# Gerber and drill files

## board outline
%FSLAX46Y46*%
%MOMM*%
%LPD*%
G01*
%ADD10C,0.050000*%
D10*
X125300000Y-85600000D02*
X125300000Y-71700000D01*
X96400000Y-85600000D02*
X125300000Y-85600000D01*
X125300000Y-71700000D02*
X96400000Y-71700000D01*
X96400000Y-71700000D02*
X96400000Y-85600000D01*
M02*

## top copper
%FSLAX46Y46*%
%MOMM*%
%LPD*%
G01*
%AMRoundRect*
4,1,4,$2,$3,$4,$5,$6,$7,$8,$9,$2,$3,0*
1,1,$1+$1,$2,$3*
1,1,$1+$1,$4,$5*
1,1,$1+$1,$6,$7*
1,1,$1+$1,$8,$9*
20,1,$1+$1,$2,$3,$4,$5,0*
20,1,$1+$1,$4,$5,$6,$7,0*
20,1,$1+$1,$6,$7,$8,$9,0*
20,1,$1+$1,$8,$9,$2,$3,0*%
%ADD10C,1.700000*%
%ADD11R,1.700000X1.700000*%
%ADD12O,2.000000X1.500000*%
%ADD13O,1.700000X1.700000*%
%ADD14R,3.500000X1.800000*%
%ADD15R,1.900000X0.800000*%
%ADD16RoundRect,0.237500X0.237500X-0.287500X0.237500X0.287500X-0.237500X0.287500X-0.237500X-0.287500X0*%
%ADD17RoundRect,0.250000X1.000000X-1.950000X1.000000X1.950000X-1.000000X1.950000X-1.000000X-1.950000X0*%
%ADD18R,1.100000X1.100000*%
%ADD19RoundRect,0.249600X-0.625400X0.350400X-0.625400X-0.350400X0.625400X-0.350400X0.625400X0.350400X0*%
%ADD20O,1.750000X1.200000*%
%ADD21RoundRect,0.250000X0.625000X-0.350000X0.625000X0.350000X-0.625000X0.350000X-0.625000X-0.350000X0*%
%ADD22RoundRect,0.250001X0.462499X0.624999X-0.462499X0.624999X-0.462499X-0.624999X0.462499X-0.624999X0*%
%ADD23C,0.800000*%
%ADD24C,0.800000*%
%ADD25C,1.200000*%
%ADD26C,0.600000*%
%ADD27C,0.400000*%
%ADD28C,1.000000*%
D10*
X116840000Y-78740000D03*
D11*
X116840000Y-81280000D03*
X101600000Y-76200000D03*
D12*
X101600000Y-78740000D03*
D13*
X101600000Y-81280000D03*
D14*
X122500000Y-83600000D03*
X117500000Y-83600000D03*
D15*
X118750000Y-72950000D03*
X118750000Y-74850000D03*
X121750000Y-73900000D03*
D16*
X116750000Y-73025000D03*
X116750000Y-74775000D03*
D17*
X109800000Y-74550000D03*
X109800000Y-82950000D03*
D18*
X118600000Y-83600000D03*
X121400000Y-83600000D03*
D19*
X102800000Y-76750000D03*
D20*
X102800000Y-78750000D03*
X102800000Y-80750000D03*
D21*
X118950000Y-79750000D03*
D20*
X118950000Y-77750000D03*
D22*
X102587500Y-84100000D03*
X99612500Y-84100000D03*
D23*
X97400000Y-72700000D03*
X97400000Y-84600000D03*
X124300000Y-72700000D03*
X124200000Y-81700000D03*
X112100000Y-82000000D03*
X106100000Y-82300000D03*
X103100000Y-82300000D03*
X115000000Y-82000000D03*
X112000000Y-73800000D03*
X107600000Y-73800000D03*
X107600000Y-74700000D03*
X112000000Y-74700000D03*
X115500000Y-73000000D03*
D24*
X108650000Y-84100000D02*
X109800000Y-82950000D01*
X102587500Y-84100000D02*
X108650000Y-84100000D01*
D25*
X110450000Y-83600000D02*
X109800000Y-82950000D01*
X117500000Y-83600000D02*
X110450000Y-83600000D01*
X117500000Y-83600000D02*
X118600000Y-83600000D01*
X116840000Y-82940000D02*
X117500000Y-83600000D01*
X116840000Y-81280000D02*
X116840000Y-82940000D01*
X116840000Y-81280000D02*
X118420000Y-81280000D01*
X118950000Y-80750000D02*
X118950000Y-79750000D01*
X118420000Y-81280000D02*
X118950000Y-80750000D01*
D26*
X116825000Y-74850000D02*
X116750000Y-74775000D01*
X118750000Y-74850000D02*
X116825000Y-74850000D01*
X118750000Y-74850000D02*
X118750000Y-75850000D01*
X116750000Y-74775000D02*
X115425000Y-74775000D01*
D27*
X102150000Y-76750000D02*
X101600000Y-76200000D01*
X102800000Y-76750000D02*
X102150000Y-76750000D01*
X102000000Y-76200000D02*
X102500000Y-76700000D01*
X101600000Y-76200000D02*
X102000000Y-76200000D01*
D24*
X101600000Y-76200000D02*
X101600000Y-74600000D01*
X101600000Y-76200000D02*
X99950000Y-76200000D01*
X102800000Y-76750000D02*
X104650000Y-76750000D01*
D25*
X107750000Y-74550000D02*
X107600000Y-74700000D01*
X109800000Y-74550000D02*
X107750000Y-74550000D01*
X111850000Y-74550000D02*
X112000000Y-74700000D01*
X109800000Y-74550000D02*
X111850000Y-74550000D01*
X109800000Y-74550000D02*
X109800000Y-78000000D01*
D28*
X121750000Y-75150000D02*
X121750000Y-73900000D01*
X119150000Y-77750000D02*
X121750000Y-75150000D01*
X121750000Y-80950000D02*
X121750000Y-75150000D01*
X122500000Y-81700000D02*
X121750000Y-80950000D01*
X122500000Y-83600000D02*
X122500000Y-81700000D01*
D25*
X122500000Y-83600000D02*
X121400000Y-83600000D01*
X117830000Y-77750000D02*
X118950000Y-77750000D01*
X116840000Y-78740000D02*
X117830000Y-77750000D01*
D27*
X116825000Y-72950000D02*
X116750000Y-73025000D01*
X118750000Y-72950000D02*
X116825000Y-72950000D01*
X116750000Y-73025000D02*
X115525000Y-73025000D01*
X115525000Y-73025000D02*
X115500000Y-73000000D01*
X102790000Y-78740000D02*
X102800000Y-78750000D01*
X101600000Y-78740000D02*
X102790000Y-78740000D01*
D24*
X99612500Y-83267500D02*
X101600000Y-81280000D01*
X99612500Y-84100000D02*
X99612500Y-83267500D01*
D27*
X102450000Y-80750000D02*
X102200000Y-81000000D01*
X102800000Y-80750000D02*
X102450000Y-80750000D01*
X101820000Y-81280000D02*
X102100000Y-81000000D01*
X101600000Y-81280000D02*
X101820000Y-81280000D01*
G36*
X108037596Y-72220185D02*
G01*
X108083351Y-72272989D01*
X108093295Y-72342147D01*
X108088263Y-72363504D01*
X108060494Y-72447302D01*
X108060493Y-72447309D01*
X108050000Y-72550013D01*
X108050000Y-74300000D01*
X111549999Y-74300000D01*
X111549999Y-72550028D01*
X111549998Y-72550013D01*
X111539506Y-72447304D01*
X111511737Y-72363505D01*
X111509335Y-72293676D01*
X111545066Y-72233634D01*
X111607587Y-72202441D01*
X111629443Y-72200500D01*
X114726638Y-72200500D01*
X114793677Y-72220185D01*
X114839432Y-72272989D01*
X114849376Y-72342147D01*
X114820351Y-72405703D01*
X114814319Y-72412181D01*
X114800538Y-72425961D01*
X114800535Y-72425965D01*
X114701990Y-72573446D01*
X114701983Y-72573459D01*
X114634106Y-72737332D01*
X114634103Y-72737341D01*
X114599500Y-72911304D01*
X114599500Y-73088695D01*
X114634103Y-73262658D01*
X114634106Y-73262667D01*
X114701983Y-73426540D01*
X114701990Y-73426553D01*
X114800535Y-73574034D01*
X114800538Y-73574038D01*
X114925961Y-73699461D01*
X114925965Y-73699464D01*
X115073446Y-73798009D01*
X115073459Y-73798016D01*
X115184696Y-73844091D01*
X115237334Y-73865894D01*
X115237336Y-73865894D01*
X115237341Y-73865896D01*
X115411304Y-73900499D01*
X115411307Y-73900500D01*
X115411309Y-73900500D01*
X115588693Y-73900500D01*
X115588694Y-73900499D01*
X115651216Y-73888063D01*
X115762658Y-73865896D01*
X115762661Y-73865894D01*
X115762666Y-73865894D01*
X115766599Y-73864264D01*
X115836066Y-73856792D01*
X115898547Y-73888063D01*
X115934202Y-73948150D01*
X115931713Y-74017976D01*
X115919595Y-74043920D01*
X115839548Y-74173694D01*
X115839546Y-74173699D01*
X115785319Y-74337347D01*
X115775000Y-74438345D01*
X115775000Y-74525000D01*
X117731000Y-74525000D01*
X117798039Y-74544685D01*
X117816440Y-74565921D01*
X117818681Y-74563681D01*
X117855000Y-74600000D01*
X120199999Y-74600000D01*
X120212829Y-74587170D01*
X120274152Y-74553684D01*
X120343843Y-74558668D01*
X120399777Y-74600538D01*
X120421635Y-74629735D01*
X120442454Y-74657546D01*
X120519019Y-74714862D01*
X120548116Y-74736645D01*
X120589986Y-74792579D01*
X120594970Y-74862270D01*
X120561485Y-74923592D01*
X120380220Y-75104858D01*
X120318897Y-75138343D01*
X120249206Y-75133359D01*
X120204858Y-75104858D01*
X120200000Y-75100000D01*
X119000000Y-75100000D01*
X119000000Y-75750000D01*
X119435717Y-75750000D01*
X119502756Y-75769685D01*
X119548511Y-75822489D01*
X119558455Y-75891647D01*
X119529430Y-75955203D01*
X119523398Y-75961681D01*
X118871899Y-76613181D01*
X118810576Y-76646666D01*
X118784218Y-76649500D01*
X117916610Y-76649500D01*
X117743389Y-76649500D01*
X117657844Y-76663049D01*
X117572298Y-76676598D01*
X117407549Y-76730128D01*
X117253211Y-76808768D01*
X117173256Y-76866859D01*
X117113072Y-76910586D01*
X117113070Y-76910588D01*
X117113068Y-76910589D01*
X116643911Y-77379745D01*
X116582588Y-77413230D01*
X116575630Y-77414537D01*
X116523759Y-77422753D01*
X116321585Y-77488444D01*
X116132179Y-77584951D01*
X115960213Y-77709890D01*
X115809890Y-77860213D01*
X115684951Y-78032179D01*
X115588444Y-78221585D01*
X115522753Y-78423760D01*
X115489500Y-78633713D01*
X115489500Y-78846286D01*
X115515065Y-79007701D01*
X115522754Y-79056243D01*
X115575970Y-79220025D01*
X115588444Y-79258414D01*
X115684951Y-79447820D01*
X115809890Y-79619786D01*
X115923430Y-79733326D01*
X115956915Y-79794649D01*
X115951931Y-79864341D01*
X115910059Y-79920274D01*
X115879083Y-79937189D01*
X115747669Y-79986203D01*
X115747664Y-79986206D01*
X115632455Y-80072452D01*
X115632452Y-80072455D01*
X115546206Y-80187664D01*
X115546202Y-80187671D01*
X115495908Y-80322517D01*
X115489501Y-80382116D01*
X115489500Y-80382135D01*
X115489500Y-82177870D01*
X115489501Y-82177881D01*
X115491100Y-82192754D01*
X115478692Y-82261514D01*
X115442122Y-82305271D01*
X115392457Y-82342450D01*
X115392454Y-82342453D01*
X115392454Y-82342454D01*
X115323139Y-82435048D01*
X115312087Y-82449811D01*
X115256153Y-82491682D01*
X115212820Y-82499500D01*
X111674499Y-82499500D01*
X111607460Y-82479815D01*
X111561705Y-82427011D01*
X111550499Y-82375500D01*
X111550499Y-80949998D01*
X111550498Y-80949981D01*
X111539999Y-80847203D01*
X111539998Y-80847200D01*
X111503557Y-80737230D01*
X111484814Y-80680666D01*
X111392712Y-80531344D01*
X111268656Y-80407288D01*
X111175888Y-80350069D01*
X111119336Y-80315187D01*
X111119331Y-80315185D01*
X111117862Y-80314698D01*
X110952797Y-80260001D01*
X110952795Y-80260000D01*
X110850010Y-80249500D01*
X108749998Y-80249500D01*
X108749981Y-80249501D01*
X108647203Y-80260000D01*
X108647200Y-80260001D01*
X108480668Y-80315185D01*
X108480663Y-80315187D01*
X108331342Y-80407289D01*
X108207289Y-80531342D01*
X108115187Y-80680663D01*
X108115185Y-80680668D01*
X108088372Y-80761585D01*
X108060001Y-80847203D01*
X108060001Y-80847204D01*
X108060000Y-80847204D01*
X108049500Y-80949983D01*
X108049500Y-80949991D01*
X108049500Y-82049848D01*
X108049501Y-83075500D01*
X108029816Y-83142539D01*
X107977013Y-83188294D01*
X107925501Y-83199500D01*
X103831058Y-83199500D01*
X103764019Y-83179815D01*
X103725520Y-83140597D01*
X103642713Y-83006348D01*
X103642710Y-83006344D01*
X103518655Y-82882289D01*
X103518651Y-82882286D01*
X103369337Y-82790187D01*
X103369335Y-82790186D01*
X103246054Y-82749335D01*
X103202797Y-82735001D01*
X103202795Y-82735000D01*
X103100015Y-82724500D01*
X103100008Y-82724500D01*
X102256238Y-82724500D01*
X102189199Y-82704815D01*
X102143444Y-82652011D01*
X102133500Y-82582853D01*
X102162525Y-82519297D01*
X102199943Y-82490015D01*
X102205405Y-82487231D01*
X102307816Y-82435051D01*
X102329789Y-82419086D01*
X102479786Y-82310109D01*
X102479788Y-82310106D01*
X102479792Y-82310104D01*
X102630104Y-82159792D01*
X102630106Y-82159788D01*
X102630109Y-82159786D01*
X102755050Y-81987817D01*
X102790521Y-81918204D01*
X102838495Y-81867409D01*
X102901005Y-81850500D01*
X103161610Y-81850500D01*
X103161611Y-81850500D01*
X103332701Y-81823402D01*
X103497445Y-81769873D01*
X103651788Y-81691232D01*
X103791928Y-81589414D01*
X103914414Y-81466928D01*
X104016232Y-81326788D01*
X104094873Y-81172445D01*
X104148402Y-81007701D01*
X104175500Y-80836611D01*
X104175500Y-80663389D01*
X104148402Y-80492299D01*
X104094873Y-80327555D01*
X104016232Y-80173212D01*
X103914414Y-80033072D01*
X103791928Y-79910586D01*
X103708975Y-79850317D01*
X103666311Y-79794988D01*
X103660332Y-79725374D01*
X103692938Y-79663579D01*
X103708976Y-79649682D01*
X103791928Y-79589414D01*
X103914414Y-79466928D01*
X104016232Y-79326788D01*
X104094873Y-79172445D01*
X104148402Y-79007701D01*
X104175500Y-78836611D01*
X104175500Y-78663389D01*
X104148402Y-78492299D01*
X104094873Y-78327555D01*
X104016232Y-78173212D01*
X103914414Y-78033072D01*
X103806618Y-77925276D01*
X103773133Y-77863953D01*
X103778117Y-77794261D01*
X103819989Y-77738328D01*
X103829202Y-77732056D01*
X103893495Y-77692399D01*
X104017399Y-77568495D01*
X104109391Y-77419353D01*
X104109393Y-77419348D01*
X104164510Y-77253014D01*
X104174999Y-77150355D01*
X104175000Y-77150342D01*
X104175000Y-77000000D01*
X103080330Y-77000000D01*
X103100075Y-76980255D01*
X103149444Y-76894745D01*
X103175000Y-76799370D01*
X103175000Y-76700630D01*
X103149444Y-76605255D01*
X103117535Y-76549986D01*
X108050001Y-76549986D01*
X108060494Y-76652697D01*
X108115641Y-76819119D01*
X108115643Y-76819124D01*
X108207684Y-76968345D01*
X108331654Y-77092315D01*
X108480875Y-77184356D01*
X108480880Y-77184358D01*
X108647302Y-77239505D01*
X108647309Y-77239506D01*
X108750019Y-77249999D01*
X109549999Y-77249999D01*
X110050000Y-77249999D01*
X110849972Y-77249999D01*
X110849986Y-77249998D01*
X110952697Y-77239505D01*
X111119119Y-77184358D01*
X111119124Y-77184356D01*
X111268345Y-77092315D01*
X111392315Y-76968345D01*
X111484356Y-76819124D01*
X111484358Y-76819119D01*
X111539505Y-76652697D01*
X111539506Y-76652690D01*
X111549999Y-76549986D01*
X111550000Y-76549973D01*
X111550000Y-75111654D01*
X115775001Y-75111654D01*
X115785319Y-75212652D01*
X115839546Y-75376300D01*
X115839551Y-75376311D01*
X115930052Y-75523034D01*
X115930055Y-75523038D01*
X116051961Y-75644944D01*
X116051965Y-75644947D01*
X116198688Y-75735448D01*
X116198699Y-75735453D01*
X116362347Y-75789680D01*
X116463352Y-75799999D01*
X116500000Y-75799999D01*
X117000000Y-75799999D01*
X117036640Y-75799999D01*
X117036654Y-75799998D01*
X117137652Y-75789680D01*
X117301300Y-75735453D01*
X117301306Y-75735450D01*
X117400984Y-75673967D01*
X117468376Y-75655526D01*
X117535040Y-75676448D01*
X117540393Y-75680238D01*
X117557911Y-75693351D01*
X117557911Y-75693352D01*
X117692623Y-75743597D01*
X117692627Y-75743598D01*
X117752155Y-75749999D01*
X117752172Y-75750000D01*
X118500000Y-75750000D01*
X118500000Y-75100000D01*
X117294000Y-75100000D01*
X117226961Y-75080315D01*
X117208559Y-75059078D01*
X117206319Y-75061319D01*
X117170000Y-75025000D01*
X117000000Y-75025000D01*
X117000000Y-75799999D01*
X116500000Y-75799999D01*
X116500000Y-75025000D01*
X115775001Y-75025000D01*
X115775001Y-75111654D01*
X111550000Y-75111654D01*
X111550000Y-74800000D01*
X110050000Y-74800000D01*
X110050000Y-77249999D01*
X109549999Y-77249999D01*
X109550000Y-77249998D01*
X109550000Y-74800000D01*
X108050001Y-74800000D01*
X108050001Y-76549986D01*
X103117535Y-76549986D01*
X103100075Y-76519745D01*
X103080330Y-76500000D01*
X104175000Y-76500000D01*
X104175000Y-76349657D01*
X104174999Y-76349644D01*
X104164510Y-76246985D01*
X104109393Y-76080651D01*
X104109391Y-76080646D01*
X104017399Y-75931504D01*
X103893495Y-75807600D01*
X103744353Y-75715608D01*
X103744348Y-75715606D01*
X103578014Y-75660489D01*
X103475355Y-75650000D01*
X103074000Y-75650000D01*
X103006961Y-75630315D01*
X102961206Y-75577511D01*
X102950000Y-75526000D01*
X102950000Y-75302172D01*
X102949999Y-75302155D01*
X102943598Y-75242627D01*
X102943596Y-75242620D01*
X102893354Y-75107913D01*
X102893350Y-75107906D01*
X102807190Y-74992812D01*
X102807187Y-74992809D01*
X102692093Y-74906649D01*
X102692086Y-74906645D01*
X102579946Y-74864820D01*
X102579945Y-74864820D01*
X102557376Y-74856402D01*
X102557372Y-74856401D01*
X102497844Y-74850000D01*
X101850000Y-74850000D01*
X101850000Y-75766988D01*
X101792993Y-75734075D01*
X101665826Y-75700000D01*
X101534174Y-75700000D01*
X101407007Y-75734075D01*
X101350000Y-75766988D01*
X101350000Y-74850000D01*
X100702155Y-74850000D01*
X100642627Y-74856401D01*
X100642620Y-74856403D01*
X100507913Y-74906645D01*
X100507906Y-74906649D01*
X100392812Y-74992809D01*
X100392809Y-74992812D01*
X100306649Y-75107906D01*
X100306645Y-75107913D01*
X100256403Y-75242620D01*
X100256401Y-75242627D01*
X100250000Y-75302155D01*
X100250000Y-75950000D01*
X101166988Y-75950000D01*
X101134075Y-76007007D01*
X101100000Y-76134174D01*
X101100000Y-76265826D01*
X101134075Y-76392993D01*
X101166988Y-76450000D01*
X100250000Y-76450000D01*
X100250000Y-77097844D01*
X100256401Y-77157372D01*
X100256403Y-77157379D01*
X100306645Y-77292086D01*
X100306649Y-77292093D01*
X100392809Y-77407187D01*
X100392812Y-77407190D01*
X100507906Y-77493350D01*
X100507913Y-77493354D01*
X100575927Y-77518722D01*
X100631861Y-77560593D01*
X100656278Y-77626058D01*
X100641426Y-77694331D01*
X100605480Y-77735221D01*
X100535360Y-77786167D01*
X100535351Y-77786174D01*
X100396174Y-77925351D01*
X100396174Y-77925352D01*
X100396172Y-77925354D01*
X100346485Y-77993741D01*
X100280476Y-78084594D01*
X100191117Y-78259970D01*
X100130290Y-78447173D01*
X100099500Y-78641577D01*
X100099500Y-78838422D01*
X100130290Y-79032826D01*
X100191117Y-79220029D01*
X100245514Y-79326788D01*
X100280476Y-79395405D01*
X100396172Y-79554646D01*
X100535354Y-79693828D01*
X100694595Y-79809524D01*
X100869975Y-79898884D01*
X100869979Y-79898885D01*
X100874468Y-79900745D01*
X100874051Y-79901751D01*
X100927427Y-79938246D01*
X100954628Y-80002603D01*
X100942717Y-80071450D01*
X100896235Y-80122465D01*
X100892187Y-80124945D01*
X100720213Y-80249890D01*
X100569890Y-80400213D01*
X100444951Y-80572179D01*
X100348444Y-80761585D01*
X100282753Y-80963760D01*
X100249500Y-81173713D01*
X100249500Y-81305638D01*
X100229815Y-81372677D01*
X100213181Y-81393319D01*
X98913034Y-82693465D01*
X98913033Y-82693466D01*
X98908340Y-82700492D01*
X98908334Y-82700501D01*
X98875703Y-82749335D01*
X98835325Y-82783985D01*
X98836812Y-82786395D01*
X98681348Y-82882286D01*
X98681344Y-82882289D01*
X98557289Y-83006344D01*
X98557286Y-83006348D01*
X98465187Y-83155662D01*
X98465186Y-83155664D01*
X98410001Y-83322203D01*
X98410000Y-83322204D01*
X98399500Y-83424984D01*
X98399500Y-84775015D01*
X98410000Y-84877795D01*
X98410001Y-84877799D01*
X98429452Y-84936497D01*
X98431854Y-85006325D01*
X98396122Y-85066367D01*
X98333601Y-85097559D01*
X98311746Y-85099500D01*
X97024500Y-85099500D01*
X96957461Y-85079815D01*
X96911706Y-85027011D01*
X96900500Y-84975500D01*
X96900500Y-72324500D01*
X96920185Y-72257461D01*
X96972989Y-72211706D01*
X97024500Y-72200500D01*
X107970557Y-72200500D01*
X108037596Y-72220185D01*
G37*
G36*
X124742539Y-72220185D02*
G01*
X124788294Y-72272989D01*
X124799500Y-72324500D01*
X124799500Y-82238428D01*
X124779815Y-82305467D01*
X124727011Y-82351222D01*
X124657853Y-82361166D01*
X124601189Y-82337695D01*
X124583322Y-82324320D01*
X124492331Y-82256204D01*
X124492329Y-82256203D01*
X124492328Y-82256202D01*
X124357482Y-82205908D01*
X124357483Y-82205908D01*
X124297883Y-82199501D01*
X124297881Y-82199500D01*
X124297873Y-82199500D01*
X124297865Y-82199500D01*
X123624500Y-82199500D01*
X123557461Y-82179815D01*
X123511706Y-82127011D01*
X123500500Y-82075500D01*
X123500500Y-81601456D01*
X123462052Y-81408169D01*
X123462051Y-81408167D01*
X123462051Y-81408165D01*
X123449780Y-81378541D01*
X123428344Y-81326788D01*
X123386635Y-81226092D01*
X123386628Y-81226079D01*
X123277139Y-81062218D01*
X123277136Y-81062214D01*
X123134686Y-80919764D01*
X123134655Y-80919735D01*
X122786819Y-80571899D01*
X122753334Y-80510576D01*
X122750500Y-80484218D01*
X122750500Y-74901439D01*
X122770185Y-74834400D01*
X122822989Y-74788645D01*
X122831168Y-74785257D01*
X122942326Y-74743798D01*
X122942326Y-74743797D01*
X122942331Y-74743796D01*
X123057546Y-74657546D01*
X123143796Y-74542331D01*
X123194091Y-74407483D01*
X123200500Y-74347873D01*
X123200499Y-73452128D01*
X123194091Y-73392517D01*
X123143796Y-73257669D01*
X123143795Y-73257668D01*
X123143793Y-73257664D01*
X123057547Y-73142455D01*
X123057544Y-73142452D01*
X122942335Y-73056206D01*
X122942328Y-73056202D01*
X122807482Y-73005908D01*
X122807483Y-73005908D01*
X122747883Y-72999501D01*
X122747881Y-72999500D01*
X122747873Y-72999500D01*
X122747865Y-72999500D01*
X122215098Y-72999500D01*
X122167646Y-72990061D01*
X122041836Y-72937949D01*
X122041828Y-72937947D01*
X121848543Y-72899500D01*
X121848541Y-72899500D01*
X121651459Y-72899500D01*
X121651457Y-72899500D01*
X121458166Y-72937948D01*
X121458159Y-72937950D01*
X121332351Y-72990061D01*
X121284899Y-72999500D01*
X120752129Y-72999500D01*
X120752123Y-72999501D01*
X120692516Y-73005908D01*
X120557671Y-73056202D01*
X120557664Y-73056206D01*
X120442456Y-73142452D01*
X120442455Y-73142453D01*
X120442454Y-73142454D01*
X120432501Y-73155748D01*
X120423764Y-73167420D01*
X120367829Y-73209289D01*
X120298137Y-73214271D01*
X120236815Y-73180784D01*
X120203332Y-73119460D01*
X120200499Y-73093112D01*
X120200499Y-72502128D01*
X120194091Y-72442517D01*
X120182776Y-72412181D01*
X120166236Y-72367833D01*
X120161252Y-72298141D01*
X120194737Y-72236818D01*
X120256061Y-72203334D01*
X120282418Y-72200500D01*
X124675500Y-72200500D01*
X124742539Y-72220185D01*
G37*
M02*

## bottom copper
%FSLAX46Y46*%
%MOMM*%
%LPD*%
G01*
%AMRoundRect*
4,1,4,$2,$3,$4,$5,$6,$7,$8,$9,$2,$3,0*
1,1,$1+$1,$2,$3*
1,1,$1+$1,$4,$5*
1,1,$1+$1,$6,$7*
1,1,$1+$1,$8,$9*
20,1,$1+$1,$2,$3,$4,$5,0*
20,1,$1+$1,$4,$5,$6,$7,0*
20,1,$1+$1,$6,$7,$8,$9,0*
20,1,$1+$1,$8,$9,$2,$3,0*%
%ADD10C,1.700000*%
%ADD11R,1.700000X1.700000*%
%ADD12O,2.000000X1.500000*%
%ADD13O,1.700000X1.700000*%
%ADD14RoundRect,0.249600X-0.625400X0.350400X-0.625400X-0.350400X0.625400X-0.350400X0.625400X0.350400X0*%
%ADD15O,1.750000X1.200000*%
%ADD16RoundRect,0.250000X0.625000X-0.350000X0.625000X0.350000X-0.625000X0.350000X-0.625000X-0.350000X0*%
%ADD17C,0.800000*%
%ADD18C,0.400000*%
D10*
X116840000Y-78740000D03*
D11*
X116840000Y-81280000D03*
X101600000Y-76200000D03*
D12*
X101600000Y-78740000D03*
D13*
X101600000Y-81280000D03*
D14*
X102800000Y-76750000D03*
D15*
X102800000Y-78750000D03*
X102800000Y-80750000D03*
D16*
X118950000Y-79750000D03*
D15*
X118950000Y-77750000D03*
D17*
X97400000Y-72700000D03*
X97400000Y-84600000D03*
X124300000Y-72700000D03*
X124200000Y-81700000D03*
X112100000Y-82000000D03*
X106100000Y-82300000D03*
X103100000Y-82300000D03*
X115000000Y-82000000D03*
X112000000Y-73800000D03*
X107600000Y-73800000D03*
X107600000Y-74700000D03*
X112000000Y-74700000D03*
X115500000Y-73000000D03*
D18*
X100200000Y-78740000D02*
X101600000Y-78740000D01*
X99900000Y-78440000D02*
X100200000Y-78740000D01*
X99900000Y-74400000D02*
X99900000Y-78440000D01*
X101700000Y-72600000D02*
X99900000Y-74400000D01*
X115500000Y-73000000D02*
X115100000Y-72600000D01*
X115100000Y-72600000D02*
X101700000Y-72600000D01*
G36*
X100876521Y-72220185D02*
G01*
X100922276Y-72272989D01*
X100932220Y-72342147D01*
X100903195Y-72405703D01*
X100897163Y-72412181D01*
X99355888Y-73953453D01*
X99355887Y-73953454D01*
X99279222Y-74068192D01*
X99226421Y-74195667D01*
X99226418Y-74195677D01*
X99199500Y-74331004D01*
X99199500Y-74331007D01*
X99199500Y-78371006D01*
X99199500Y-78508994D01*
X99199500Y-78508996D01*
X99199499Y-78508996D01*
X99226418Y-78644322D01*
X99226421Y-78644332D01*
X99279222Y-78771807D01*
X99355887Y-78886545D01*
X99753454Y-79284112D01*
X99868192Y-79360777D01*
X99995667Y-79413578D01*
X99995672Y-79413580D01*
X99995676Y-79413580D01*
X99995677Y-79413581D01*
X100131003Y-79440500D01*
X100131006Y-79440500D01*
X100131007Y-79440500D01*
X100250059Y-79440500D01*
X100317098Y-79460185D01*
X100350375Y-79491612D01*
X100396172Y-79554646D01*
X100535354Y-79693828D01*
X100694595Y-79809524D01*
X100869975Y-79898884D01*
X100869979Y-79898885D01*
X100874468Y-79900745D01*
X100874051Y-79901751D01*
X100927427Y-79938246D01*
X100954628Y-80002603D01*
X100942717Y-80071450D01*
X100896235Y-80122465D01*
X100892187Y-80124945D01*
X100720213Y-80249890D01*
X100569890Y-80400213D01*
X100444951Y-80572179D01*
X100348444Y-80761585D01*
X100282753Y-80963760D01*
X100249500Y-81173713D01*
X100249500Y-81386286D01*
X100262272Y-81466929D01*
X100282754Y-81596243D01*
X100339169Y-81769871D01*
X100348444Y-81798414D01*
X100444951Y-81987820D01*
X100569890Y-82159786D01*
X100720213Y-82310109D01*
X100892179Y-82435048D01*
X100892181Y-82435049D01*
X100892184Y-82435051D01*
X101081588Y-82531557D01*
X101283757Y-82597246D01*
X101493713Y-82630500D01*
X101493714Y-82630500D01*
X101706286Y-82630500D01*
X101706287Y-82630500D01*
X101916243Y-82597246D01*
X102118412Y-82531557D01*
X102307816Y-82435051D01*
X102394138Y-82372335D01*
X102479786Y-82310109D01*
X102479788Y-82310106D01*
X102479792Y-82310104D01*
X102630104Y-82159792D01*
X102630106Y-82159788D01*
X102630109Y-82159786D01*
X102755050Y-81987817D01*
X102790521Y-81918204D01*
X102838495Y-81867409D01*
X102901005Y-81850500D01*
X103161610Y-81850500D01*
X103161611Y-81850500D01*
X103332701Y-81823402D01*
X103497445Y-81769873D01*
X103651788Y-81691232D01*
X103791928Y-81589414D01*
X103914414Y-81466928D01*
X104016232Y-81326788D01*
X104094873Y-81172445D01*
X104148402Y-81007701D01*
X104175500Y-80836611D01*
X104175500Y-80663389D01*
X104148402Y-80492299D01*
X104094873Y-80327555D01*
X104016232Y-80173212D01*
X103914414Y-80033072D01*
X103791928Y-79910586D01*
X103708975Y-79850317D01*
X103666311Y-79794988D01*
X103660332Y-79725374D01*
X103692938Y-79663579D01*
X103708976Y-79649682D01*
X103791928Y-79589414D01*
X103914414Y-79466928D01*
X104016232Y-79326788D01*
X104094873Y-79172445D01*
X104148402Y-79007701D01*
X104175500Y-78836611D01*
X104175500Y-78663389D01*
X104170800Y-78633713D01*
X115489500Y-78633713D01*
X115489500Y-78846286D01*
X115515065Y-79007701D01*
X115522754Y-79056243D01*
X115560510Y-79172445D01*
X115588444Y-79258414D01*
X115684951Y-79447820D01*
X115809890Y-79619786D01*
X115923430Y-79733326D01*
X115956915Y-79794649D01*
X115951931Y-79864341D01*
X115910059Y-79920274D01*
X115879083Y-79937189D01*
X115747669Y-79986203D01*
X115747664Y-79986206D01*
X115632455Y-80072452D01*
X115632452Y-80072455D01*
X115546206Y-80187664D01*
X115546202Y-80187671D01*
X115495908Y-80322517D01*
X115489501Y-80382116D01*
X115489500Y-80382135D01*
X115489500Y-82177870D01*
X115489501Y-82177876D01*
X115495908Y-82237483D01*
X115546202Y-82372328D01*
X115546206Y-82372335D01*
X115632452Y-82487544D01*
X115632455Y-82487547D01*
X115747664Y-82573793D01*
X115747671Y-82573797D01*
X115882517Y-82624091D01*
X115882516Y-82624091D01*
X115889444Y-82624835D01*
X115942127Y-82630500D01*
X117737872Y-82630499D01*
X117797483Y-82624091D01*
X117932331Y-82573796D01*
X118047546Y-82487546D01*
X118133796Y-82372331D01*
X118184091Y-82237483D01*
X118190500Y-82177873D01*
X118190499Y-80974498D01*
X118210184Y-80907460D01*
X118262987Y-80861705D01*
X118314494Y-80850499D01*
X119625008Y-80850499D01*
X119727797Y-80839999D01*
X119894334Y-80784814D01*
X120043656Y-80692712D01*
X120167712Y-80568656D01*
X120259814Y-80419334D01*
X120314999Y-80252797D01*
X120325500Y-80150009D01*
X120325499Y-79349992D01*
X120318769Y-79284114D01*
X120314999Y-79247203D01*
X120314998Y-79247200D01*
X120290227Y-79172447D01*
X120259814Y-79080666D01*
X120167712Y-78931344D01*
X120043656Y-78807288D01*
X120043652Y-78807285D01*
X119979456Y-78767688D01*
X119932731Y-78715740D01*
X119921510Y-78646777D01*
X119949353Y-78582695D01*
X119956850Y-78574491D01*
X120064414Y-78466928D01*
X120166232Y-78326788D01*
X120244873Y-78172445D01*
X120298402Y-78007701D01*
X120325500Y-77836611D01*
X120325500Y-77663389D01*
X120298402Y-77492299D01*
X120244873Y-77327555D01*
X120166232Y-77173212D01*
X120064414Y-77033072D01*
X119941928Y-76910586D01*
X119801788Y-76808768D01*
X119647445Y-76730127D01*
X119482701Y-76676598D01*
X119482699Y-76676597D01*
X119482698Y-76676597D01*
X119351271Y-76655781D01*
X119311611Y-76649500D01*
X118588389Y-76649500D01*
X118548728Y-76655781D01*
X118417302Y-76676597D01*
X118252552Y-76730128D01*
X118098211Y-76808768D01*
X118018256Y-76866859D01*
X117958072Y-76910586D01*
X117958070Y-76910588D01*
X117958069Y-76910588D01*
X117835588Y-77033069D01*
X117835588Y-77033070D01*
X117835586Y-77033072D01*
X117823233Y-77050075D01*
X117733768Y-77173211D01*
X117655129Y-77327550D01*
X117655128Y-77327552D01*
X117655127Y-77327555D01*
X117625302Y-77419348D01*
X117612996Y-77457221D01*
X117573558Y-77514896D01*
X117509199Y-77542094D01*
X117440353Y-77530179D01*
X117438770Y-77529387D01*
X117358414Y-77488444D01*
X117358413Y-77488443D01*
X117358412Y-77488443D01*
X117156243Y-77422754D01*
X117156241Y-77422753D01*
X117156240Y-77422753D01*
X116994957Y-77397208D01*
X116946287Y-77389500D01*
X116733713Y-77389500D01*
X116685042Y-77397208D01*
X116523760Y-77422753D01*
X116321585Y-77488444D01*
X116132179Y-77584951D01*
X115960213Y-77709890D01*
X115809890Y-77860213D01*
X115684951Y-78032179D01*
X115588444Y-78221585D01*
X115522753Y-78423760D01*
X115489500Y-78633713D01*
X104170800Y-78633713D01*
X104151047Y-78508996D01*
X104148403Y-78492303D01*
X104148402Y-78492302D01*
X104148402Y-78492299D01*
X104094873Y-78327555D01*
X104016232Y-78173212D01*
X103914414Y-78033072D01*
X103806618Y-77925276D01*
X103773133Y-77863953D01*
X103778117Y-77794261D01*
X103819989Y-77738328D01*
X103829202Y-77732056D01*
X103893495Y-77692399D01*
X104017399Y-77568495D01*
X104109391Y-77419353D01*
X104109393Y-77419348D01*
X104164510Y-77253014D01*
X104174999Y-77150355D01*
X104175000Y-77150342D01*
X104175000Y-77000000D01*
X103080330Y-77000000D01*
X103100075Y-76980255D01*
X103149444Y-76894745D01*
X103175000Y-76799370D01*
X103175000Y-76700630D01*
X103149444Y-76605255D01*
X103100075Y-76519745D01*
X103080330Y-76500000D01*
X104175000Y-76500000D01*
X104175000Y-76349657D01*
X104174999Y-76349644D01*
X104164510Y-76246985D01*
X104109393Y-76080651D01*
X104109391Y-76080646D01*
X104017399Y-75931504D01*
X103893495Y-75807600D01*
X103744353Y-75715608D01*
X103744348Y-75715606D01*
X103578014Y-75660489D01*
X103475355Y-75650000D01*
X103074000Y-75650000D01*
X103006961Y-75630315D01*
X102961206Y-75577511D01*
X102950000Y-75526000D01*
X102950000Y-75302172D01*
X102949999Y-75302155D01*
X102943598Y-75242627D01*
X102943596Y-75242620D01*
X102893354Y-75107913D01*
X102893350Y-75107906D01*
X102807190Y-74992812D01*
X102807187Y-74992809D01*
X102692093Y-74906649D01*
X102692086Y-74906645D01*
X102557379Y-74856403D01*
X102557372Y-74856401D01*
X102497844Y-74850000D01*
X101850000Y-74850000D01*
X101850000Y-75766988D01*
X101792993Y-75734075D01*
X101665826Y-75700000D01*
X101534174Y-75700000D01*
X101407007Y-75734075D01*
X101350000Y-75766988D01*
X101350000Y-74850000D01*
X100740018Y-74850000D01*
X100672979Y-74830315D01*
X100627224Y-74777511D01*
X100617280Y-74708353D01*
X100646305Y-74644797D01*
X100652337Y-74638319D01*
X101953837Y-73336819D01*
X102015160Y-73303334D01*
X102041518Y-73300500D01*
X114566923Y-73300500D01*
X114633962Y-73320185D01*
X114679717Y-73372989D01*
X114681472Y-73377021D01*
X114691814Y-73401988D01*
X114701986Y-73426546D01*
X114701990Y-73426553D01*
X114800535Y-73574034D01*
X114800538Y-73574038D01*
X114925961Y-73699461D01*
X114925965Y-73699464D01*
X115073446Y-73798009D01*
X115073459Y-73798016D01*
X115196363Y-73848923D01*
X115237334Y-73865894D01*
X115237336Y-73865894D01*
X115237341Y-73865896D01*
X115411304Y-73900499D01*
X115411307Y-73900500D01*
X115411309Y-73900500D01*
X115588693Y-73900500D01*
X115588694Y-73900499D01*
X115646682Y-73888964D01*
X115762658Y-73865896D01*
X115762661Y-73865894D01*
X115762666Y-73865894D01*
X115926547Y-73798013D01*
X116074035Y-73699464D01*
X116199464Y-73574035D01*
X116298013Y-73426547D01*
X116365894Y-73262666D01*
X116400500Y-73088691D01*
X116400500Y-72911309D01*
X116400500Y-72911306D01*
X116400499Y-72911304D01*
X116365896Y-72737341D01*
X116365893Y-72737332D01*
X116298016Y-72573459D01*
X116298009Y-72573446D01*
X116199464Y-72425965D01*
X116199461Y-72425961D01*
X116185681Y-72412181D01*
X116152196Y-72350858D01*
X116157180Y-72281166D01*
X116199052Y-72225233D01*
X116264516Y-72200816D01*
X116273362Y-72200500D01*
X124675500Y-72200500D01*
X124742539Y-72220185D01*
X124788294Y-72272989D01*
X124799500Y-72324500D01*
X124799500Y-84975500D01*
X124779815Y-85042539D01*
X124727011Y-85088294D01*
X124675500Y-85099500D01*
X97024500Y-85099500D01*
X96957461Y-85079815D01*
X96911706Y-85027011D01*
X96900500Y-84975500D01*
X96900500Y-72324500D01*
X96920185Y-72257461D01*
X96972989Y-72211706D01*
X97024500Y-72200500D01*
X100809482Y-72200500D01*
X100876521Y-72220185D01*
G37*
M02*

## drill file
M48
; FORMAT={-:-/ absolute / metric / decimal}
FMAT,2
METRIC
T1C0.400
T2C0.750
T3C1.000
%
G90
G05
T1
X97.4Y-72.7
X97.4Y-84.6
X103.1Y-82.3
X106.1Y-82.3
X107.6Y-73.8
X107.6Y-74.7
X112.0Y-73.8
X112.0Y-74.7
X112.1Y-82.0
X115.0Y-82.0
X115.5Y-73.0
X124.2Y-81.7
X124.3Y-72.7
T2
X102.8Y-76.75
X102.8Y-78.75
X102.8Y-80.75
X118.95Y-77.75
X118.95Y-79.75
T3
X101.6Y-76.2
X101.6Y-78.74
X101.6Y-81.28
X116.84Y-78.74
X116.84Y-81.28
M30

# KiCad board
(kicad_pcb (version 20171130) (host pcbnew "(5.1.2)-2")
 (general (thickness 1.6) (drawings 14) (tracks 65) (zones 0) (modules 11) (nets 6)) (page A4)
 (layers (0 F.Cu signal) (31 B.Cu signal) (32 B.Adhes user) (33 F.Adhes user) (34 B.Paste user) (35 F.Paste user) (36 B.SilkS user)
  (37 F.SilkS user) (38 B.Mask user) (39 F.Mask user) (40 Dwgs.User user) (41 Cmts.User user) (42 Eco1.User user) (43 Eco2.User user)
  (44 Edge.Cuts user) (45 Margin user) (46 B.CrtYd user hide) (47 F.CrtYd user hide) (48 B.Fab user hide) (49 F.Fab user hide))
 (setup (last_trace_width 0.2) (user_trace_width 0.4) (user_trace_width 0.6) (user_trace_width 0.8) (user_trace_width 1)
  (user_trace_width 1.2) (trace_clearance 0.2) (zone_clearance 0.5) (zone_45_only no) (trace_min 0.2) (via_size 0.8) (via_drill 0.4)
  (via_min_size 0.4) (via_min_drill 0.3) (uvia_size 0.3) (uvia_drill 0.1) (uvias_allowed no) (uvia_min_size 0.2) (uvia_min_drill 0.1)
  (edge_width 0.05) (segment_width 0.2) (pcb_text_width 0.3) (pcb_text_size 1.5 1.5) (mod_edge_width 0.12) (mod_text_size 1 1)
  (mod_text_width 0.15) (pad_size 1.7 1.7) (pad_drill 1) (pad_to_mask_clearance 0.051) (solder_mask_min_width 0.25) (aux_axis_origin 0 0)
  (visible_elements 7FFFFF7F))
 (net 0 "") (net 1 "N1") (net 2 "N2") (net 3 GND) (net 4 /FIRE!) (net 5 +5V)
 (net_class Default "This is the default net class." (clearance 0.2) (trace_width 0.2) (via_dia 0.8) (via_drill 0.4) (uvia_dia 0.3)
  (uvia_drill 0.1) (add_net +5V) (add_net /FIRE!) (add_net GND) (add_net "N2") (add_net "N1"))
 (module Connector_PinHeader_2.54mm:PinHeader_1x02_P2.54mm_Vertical (layer F.Cu) (at 116.84 81.28 180)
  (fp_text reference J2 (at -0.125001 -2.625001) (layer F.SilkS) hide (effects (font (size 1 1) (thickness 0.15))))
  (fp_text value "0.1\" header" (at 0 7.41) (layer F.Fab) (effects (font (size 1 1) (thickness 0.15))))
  (pad 2 thru_hole circle (at 0 2.54 180) (size 1.7 1.7) (drill 1) (layers *.Cu *.Mask) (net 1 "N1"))
  (pad 1 thru_hole rect (at 0 0 180) (size 1.7 1.7) (drill 1) (layers *.Cu *.Mask) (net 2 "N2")))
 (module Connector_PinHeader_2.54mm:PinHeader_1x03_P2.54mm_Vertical (layer F.Cu) (at 101.6 76.2)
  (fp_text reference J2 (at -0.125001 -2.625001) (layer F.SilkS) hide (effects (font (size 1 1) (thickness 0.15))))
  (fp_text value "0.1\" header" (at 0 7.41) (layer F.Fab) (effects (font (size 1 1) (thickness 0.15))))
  (pad 1 thru_hole rect (at 0 0 90) (size 1.7 1.7) (drill 1) (layers *.Cu *.Mask) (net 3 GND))
  (pad 2 thru_hole oval (at 0 2.54) (size 2 1.5) (drill 1) (layers *.Cu *.Mask) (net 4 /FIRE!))
  (pad 3 thru_hole oval (at 0 5.08) (size 1.7 1.7) (drill 1) (layers *.Cu *.Mask) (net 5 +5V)))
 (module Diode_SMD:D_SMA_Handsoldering (layer F.Cu) (at 120 83.6)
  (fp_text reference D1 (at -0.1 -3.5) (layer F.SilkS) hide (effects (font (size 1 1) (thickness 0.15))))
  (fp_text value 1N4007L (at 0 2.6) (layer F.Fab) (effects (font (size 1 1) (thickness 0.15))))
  (pad 2 smd rect (at 2.5 0) (size 3.5 1.8) (layers F.Cu F.Paste F.Mask) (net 1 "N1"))
  (pad 1 smd rect (at -2.5 0) (size 3.5 1.8) (layers F.Cu F.Paste F.Mask) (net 2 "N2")))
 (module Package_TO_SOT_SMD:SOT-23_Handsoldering (layer F.Cu) (at 120.25 73.9)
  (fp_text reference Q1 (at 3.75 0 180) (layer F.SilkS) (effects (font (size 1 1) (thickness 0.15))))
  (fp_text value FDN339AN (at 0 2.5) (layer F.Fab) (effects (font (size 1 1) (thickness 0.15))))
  (pad 1 smd rect (at -1.5 -0.95) (size 1.9 0.8) (layers F.Cu F.Paste F.Mask) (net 4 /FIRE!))
  (pad 2 smd rect (at -1.5 0.95) (size 1.9 0.8) (layers F.Cu F.Paste F.Mask) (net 3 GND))
  (pad 3 smd rect (at 1.5 0) (size 1.9 0.8) (layers F.Cu F.Paste F.Mask) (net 1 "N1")))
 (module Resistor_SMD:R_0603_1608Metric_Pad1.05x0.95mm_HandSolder (layer F.Cu) (at 116.75 73.9 90)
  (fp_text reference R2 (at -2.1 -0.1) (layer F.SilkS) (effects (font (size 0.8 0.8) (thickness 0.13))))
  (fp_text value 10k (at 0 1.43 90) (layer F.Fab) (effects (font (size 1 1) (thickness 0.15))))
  (pad 2 smd roundrect (at 0.875 0 90) (size 1.05 0.95) (layers F.Cu F.Paste F.Mask) (roundrect_rratio 0.25) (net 4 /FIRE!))
  (pad 1 smd roundrect (at -0.875 0 90) (size 1.05 0.95) (layers F.Cu F.Paste F.Mask) (roundrect_rratio 0.25) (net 3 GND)))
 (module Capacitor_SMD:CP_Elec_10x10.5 (layer F.Cu) (at 109.8 78.75 90)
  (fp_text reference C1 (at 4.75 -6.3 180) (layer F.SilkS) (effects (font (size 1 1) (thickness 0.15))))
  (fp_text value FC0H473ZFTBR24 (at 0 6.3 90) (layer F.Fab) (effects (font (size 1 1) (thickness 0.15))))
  (pad 2 smd roundrect (at 4.2 0 90) (size 4.4 2.5) (layers F.Cu F.Paste F.Mask) (roundrect_rratio 0.1) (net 3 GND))
  (pad 1 smd roundrect (at -4.2 0 90) (size 4.4 2.5) (layers F.Cu F.Paste F.Mask) (roundrect_rratio 0.1) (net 2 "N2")))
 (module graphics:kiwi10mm (layer B.Cu) (at 109.6 79.1 180)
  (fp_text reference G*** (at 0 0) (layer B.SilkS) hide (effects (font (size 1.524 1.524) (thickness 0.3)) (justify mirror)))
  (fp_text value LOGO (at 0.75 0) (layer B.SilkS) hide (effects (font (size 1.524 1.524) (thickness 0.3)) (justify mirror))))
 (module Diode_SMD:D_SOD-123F (layer F.Cu) (at 120 83.6)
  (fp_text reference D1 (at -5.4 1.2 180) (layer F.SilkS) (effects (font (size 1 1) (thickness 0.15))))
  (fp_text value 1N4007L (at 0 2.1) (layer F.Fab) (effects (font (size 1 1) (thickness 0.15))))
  (pad 1 smd rect (at -1.4 0) (size 1.1 1.1) (layers F.Cu F.Paste F.Mask) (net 2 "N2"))
  (pad 2 smd rect (at 1.4 0) (size 1.1 1.1) (layers F.Cu F.Paste F.Mask) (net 1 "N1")))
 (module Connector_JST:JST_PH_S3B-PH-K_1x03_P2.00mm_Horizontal (layer F.Cu) (at 102.8 76.75 270)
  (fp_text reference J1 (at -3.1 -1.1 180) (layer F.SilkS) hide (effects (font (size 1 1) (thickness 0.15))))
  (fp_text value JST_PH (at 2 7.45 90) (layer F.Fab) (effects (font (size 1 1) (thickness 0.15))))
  (pad 1 thru_hole roundrect (at 0 0 270) (size 1.2 1.75) (drill 0.75) (layers *.Cu *.Mask) (roundrect_rratio 0.208) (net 3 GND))
  (pad 2 thru_hole oval (at 2 0 270) (size 1.2 1.75) (drill 0.75) (layers *.Cu *.Mask) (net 4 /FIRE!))
  (pad 3 thru_hole oval (at 4 0 270) (size 1.2 1.75) (drill 0.75) (layers *.Cu *.Mask) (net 5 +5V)))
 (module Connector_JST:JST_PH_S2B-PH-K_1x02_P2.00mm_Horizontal (layer F.Cu) (at 118.95 79.75 90)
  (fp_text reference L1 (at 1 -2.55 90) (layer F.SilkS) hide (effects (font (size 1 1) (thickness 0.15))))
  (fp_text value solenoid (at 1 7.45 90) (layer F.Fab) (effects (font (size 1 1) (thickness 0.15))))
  (pad 1 thru_hole roundrect (at 0 0 90) (size 1.2 1.75) (drill 0.75) (layers *.Cu *.Mask) (roundrect_rratio 0.208333) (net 2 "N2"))
  (pad 2 thru_hole oval (at 2 0 90) (size 1.2 1.75) (drill 0.75) (layers *.Cu *.Mask) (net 1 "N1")))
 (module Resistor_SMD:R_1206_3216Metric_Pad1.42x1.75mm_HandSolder (layer F.Cu) (at 101.1 84.1 180)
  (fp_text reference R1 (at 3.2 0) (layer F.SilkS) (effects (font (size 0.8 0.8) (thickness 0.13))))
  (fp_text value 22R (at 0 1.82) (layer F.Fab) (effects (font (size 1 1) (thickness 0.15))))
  (pad 1 smd roundrect (at -1.4875 0 180) (size 1.425 1.75) (layers F.Cu F.Paste F.Mask) (roundrect_rratio 0.175439) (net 2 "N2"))
  (pad 2 smd roundrect (at 1.4875 0 180) (size 1.425 1.75) (layers F.Cu F.Paste F.Mask) (roundrect_rratio 0.175439) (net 5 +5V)))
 (gr_line (start 125.3 85.6) (end 125.3 71.7) (layer Edge.Cuts) (width 0.05))
 (gr_line (start 96.4 85.6) (end 125.3 85.6) (layer Edge.Cuts) (width 0.05))
 (gr_line (start 125.3 71.7) (end 96.4 71.7) (layer Edge.Cuts) (width 0.05))
 (gr_line (start 96.4 71.7) (end 96.4 85.6) (layer Edge.Cuts) (width 0.05))
 (segment (start 108.65 84.1) (end 109.8 82.95) (width 0.8) (layer F.Cu) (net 2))
 (segment (start 102.5875 84.1) (end 108.65 84.1) (width 0.8) (layer F.Cu) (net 2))
 (segment (start 110.45 83.6) (end 109.8 82.95) (width 1.2) (layer F.Cu) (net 2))
 (segment (start 117.5 83.6) (end 110.45 83.6) (width 1.2) (layer F.Cu) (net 2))
 (segment (start 117.5 83.6) (end 118.6 83.6) (width 1.2) (layer F.Cu) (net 2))
 (segment (start 116.84 82.94) (end 117.5 83.6) (width 1.2) (layer F.Cu) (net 2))
 (segment (start 116.84 81.28) (end 116.84 82.94) (width 1.2) (layer F.Cu) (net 2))
 (segment (start 116.84 81.28) (end 118.42 81.28) (width 1.2) (layer F.Cu) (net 2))
 (segment (start 118.95 80.75) (end 118.95 79.75) (width 1.2) (layer F.Cu) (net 2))
 (segment (start 118.42 81.28) (end 118.95 80.75) (width 1.2) (layer F.Cu) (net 2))
 (segment (start 116.825 74.85) (end 116.75 74.775) (width 0.6) (layer F.Cu) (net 3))
 (segment (start 118.75 74.85) (end 116.825 74.85) (width 0.6) (layer F.Cu) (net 3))
 (segment (start 118.75 74.85) (end 118.75 75.85) (width 0.6) (layer F.Cu) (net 3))
 (segment (start 116.75 74.775) (end 115.425 74.775) (width 0.6) (layer F.Cu) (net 3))
 (segment (start 102.15 76.75) (end 101.6 76.2) (width 0.4) (layer F.Cu) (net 3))
 (segment (start 102.8 76.75) (end 102.15 76.75) (width 0.4) (layer F.Cu) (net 3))
 (via (at 97.4 72.7) (size 0.8) (drill 0.4) (layers F.Cu B.Cu) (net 3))
 (via (at 97.4 84.6) (size 0.8) (drill 0.4) (layers F.Cu B.Cu) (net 3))
 (via (at 124.3 72.7) (size 0.8) (drill 0.4) (layers F.Cu B.Cu) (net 3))
 (via (at 124.2 81.7) (size 0.8) (drill 0.4) (layers F.Cu B.Cu) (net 3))
 (via (at 112.1 82) (size 0.8) (drill 0.4) (layers F.Cu B.Cu) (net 3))
 (via (at 106.1 82.3) (size 0.8) (drill 0.4) (layers F.Cu B.Cu) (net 3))
 (via (at 103.1 82.3) (size 0.8) (drill 0.4) (layers F.Cu B.Cu) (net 3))
 (segment (start 102 76.2) (end 102.5 76.7) (width 0.4) (layer F.Cu) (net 3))
 (segment (start 101.6 76.2) (end 102 76.2) (width 0.4) (layer F.Cu) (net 3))
 (segment (start 101.6 76.2) (end 101.6 74.6) (width 0.8) (layer F.Cu) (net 3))
 (segment (start 101.6 76.2) (end 99.95 76.2) (width 0.8) (layer F.Cu) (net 3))
 (segment (start 102.8 76.75) (end 104.65 76.75) (width 0.8) (layer F.Cu) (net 3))
 (via (at 115 82) (size 0.8) (drill 0.4) (layers F.Cu B.Cu) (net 3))
 (via (at 112 73.8) (size 0.8) (drill 0.4) (layers F.Cu B.Cu) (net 3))
 (via (at 107.6 73.8) (size 0.8) (drill 0.4) (layers F.Cu B.Cu) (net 3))
 (via (at 107.6 74.7) (size 0.8) (drill 0.4) (layers F.Cu B.Cu) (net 3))
 (via (at 112 74.7) (size 0.8) (drill 0.4) (layers F.Cu B.Cu) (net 3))
 (segment (start 107.75 74.55) (end 107.6 74.7) (width 1.2) (layer F.Cu) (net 3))
 (segment (start 109.8 74.55) (end 107.75 74.55) (width 1.2) (layer F.Cu) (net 3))
 (segment (start 111.85 74.55) (end 112 74.7) (width 1.2) (layer F.Cu) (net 3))
 (segment (start 109.8 74.55) (end 111.85 74.55) (width 1.2) (layer F.Cu) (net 3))
 (segment (start 109.8 74.55) (end 109.8 78) (width 1.2) (layer F.Cu) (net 3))
 (segment (start 121.75 75.15) (end 121.75 73.9) (width 1) (layer F.Cu) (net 1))
 (segment (start 119.15 77.75) (end 121.75 75.15) (width 1) (layer F.Cu) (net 1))
 (segment (start 121.75 80.95) (end 121.75 75.15) (width 1) (layer F.Cu) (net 1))
 (segment (start 122.5 81.7) (end 121.75 80.95) (width 1) (layer F.Cu) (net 1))
 (segment (start 122.5 83.6) (end 122.5 81.7) (width 1) (layer F.Cu) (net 1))
 (segment (start 122.5 83.6) (end 121.4 83.6) (width 1.2) (layer F.Cu) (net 1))
 (segment (start 117.83 77.75) (end 118.95 77.75) (width 1.2) (layer F.Cu) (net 1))
 (segment (start 116.84 78.74) (end 117.83 77.75) (width 1.2) (layer F.Cu) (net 1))
 (segment (start 116.825 72.95) (end 116.75 73.025) (width 0.4) (layer F.Cu) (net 4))
 (segment (start 118.75 72.95) (end 116.825 72.95) (width 0.4) (layer F.Cu) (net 4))
 (via (at 115.5 73) (size 0.8) (drill 0.4) (layers F.Cu B.Cu) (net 4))
 (segment (start 116.75 73.025) (end 115.525 73.025) (width 0.4) (layer F.Cu) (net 4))
 (segment (start 115.525 73.025) (end 115.5 73) (width 0.4) (layer F.Cu) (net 4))
 (segment (start 102.79 78.74) (end 102.8 78.75) (width 0.4) (layer F.Cu) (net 4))
 (segment (start 101.6 78.74) (end 102.79 78.74) (width 0.4) (layer F.Cu) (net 4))
 (segment (start 100.2 78.74) (end 101.6 78.74) (width 0.4) (layer B.Cu) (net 4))
 (segment (start 99.9 78.44) (end 100.2 78.74) (width 0.4) (layer B.Cu) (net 4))
 (segment (start 99.9 74.4) (end 99.9 78.44) (width 0.4) (layer B.Cu) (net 4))
 (segment (start 101.7 72.6) (end 99.9 74.4) (width 0.4) (layer B.Cu) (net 4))
 (segment (start 115.5 73) (end 115.1 72.6) (width 0.4) (layer B.Cu) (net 4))
 (segment (start 115.1 72.6) (end 101.7 72.6) (width 0.4) (layer B.Cu) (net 4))
 (segment (start 99.6125 83.2675) (end 101.6 81.28) (width 0.8) (layer F.Cu) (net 5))
 (segment (start 99.6125 84.1) (end 99.6125 83.2675) (width 0.8) (layer F.Cu) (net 5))
 (segment (start 102.45 80.75) (end 102.2 81) (width 0.4) (layer F.Cu) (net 5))
 (segment (start 102.8 80.75) (end 102.45 80.75) (width 0.4) (layer F.Cu) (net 5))
 (segment (start 101.82 81.28) (end 102.1 81) (width 0.4) (layer F.Cu) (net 5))
 (segment (start 101.6 81.28) (end 101.82 81.28) (width 0.4) (layer F.Cu) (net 5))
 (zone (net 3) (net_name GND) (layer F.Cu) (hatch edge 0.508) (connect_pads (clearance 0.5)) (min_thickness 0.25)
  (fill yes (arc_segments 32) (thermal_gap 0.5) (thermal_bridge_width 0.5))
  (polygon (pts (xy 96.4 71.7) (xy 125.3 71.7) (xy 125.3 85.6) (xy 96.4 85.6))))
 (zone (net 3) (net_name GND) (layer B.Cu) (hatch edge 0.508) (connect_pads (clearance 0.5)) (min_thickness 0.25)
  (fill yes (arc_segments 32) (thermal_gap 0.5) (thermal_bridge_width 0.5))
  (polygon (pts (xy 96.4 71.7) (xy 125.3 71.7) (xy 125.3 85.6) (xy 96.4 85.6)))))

